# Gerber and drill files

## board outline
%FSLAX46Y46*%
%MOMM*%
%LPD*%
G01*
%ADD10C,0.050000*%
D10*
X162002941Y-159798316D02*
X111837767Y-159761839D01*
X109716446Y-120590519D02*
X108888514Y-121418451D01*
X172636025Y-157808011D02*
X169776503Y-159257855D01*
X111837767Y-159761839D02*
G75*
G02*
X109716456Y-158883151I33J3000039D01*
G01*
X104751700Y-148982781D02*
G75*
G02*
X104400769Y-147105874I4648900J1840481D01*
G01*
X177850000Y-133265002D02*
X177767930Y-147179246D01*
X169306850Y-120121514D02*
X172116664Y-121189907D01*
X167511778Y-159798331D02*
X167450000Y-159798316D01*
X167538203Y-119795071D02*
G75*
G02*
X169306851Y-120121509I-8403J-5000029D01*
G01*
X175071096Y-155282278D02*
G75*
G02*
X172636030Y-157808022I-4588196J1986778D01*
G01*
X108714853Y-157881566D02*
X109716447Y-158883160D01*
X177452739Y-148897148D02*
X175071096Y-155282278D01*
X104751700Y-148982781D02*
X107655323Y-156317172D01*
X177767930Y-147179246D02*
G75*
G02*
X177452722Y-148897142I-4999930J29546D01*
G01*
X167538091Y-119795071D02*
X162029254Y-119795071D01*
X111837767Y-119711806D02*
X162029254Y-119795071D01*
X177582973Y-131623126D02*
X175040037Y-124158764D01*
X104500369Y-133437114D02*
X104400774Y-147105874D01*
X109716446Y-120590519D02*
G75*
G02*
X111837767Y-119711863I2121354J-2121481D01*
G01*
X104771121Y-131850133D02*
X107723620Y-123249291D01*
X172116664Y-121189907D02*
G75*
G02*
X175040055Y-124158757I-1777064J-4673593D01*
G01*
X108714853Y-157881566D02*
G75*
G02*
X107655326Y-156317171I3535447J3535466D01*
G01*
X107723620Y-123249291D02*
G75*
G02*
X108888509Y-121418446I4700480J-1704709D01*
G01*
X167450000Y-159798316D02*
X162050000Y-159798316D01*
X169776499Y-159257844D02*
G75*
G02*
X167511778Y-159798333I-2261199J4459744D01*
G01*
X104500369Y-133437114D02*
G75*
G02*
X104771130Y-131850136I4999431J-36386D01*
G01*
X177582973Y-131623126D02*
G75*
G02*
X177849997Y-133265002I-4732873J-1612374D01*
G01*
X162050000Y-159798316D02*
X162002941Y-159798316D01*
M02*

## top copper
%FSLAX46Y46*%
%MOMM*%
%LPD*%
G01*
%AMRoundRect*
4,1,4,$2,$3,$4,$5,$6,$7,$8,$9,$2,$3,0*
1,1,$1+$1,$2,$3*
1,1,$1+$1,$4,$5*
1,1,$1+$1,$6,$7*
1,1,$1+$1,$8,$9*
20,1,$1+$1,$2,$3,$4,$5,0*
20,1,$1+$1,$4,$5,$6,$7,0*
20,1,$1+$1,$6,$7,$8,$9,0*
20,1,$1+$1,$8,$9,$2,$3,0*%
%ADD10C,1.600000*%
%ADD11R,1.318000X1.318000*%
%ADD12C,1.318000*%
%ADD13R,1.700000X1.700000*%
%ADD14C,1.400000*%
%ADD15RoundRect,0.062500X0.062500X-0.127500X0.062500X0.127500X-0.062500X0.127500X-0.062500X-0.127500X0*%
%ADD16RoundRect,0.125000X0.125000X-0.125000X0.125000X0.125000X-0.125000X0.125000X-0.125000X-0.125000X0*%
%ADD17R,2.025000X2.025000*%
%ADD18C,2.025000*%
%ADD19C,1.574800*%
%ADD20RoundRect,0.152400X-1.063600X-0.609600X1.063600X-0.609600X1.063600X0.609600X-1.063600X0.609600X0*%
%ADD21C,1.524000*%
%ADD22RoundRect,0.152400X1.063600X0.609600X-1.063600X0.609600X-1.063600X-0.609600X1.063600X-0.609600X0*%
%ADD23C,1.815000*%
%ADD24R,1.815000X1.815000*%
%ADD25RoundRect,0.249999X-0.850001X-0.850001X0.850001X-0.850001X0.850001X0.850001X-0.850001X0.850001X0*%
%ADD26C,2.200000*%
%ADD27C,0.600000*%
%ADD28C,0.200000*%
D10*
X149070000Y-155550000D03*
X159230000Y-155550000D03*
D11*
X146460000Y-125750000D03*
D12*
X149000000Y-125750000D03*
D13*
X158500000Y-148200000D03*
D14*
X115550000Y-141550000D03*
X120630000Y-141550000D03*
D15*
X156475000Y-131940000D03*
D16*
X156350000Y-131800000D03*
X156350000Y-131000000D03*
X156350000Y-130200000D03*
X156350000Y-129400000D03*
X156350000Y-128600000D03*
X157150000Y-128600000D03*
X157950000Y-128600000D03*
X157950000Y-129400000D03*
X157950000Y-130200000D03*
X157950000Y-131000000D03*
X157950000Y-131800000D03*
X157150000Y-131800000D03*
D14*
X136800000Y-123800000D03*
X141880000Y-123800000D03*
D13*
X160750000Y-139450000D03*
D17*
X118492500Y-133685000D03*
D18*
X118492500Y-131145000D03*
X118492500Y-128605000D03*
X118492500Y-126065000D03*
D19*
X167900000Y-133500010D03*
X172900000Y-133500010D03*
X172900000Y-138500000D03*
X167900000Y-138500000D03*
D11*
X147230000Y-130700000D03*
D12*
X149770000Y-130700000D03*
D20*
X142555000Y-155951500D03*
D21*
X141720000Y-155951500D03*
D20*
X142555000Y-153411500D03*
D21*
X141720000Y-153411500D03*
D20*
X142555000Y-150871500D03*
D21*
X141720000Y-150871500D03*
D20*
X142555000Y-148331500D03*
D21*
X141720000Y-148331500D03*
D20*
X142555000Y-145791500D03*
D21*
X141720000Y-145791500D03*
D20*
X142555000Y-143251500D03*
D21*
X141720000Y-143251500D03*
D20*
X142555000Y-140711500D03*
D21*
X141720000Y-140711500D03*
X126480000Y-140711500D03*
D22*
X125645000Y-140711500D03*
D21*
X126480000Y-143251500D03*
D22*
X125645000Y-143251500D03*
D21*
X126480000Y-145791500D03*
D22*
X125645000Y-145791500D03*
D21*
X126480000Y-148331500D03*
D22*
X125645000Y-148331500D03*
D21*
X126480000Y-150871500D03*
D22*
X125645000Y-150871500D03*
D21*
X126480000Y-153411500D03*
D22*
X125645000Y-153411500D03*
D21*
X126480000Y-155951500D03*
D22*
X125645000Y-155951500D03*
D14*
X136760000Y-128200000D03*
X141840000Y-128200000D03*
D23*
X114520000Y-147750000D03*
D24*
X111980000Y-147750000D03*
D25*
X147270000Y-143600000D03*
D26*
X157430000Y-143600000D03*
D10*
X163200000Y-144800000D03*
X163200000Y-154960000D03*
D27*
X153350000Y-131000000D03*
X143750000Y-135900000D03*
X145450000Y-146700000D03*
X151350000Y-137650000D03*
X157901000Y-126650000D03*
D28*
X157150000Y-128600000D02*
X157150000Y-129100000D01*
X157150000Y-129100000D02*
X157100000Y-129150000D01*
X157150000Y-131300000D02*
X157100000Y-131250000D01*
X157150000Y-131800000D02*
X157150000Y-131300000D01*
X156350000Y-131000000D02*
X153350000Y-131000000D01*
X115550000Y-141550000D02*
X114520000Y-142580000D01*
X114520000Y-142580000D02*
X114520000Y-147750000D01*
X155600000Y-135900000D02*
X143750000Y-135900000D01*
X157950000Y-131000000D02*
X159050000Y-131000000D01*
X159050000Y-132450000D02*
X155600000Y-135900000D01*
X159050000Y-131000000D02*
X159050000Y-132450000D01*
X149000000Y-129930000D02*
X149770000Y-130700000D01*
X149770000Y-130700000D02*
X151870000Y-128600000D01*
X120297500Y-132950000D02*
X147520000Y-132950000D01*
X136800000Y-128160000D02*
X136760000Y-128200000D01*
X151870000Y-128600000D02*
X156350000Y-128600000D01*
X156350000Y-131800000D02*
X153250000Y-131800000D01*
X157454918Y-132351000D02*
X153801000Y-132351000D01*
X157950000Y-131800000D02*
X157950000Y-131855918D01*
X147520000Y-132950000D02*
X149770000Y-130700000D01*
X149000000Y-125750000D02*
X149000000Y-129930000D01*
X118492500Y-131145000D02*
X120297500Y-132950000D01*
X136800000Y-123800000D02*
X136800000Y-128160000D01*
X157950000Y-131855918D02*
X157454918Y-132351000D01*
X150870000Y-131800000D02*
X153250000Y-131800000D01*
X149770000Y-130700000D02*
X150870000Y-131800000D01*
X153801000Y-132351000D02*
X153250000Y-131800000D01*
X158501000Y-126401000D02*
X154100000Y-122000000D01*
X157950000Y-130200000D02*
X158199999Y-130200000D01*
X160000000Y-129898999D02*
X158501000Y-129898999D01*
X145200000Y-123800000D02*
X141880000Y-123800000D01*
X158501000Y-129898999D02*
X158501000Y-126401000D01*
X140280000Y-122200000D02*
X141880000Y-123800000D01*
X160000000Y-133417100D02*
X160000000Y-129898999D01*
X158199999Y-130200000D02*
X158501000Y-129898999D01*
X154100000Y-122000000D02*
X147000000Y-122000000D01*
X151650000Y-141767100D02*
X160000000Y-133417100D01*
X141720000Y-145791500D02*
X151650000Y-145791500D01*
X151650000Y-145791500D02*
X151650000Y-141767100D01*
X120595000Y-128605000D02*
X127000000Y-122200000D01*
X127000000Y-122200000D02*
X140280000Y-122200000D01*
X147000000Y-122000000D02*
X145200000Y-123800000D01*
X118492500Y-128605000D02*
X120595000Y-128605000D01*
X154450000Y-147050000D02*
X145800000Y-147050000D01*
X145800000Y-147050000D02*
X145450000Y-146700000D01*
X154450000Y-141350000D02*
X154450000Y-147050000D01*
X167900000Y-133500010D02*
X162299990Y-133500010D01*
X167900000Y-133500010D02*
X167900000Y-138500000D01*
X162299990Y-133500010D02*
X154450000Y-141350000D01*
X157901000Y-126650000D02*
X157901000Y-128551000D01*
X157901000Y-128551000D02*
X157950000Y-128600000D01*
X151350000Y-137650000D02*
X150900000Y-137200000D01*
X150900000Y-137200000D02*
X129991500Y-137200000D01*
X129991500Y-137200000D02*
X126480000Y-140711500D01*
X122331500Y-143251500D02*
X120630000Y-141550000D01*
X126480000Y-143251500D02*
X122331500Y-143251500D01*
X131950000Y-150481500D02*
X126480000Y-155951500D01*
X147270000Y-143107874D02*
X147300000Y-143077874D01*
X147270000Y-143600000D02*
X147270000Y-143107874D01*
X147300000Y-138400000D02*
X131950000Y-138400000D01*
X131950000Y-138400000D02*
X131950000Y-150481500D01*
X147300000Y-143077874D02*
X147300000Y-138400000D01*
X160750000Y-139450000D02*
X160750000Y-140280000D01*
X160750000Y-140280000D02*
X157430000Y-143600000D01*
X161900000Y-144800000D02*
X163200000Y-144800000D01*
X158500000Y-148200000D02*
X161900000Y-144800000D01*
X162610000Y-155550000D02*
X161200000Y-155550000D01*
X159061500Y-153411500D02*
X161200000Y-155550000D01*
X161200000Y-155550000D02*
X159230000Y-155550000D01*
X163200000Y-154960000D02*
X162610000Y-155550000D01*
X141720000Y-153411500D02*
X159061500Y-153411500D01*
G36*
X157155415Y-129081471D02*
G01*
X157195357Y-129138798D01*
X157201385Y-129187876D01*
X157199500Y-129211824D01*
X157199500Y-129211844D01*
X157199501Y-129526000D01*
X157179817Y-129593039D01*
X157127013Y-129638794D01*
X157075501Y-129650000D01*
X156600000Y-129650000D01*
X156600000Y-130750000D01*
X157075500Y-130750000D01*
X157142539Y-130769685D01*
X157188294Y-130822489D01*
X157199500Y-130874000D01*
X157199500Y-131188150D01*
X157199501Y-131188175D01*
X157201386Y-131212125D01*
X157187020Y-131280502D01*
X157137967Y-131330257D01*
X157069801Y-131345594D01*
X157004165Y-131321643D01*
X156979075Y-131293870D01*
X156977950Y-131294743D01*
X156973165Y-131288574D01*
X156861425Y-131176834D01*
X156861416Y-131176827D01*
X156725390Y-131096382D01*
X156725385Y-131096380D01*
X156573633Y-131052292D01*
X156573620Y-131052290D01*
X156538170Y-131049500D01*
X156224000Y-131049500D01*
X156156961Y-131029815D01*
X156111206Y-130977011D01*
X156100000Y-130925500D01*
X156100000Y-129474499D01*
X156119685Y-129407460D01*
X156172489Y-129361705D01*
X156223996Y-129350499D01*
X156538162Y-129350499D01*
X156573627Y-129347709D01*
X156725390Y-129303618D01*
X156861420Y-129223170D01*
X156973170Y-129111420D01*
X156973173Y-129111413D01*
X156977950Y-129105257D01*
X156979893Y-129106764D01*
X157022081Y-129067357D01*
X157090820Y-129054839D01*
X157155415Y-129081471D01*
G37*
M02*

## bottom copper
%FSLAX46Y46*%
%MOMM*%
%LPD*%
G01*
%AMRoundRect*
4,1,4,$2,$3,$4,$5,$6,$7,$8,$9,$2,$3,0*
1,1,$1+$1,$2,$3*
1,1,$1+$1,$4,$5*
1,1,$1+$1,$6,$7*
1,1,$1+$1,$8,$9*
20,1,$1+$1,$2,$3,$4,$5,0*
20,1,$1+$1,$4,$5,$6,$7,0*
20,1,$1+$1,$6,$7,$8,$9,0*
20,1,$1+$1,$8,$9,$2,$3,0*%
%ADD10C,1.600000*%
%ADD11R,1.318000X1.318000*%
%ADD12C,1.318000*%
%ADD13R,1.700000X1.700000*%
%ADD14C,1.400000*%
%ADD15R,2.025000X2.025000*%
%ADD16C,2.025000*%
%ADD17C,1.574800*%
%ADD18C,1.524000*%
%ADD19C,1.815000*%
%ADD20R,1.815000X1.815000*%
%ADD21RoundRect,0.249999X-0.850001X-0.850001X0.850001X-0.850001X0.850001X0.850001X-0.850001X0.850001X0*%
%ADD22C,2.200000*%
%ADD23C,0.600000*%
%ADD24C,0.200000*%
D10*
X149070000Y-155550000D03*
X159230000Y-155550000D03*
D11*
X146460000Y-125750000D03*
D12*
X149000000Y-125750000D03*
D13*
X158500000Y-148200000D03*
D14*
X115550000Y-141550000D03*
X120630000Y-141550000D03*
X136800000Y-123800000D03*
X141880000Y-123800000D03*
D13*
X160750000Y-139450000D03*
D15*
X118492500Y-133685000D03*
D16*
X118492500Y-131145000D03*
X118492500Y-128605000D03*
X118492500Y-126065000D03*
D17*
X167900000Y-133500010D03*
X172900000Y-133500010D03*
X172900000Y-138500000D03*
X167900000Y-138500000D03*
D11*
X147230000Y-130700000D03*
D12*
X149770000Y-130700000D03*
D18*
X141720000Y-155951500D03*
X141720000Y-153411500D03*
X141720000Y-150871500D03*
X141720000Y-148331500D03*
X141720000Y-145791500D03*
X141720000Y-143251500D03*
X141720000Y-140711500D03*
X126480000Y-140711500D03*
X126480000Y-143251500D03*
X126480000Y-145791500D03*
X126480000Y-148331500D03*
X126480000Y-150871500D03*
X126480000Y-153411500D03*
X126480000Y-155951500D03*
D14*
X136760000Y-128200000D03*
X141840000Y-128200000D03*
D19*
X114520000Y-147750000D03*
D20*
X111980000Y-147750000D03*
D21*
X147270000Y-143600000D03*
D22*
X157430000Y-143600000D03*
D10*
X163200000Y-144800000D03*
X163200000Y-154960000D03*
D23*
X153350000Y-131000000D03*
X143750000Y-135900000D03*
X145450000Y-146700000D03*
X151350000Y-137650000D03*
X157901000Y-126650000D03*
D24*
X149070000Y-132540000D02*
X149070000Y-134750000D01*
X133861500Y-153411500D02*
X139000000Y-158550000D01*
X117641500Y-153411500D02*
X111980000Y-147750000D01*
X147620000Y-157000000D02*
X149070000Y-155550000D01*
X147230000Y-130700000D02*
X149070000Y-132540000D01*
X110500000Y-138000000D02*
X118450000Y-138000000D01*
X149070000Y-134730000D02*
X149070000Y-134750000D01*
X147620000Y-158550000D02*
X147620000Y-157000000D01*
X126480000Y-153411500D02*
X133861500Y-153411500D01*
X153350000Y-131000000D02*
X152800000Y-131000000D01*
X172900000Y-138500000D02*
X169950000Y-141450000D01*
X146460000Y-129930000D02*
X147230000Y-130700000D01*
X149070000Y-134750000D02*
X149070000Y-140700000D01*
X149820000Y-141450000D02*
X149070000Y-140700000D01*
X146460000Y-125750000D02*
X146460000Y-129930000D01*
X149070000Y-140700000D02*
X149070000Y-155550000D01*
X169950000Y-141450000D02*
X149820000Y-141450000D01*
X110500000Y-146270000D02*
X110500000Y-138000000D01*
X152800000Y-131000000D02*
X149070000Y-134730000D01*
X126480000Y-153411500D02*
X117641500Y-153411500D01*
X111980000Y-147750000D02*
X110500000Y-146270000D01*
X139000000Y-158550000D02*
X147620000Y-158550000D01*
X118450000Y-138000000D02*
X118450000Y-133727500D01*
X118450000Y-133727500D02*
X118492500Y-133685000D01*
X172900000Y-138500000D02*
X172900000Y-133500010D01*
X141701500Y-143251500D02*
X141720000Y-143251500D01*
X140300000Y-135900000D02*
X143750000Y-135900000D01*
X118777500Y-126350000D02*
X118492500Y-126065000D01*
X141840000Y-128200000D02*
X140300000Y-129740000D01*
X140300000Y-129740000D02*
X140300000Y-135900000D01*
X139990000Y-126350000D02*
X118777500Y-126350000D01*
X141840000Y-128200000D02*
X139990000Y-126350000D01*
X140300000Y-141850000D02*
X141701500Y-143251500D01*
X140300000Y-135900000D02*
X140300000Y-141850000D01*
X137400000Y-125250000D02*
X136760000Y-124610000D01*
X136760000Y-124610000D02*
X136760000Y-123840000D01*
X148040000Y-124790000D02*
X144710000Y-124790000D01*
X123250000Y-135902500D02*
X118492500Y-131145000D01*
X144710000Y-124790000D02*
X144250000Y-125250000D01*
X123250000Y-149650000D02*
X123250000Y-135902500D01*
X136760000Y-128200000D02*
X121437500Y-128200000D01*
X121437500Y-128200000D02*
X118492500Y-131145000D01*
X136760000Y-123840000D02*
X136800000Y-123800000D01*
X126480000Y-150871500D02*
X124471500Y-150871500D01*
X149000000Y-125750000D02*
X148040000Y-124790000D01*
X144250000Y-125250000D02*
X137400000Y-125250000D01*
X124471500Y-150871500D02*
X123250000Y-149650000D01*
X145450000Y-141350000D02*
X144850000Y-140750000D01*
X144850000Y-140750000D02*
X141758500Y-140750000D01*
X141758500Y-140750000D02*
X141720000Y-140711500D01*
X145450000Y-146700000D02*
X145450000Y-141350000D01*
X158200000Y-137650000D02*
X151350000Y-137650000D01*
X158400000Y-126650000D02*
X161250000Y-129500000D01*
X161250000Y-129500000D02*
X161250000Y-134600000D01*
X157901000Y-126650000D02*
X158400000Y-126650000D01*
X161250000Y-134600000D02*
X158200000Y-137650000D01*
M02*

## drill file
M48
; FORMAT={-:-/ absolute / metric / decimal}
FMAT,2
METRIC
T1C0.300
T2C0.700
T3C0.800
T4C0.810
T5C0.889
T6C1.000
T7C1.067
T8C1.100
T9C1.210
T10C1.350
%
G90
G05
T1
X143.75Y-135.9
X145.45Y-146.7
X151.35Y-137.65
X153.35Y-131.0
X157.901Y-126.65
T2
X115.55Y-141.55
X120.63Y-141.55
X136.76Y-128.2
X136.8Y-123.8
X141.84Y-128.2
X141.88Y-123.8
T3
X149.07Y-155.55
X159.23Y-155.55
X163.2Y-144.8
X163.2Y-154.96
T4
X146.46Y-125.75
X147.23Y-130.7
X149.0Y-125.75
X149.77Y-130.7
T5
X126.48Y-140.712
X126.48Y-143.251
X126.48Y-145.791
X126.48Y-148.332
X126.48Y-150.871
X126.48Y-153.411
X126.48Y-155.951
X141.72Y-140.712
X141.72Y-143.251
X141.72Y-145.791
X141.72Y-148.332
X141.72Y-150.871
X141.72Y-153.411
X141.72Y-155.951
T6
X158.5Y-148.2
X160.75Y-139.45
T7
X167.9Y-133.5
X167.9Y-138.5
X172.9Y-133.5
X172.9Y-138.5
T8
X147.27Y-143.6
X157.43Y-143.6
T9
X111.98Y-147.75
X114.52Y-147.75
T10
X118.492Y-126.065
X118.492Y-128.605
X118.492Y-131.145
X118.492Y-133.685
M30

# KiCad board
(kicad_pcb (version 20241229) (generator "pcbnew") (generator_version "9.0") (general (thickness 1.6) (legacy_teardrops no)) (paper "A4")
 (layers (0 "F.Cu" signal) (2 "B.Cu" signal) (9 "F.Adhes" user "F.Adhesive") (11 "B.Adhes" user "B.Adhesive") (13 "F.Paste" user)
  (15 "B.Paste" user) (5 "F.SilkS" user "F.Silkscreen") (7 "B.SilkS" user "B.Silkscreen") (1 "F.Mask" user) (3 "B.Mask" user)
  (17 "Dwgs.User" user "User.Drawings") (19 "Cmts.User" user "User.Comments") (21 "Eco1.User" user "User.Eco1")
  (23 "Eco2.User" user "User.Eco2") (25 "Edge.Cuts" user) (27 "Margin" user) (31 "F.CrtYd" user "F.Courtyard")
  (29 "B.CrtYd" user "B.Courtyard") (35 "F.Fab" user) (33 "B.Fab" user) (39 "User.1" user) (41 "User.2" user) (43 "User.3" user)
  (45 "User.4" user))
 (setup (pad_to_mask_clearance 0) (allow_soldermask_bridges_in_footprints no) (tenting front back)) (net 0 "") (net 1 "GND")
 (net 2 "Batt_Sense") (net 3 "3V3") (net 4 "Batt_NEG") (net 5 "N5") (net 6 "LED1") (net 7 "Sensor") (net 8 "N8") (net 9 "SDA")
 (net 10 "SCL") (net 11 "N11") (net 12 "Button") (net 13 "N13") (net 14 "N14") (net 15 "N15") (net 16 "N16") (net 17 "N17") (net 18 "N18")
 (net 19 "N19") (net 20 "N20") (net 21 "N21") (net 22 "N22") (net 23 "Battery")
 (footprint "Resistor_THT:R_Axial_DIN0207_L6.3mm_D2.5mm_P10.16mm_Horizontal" (layer "F.Cu") (at 149.07 155.55)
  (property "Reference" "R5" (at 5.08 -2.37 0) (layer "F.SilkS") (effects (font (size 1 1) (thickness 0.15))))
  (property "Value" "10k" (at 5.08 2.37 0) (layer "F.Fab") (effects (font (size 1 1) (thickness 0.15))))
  (pad "1" thru_hole circle (at 0 0) (size 1.6 1.6) (drill 0.8) (layers "*.Cu" "*.Mask") (remove_unused_layers no) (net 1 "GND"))
  (pad "2" thru_hole circle (at 10.16 0) (size 1.6 1.6) (drill 0.8) (layers "*.Cu" "*.Mask") (remove_unused_layers no) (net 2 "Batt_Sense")))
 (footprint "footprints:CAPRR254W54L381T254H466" (layer "F.Cu") (at 147.73 125.75)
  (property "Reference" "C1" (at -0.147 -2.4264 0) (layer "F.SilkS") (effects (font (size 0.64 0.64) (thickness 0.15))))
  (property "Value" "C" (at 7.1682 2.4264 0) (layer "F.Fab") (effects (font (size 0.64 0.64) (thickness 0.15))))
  (pad "1" thru_hole rect (at -1.27 0) (size 1.318 1.318) (drill 0.81) (layers "*.Cu" "*.Mask") (remove_unused_layers no) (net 1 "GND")
   (solder_mask_margin 0.102))
  (pad "2" thru_hole circle (at 1.27 0) (size 1.318 1.318) (drill 0.81) (layers "*.Cu" "*.Mask") (remove_unused_layers no) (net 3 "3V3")
   (solder_mask_margin 0.102)))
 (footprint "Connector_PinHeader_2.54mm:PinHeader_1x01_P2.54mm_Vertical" (layer "F.Cu") (at 158.5 148.2)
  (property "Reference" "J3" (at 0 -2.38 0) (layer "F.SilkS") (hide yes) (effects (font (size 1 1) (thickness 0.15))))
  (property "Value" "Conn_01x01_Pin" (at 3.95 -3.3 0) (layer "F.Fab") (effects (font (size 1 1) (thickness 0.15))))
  (pad "1" thru_hole rect (at 0 0) (size 1.7 1.7) (drill 1) (layers "*.Cu" "*.Mask") (remove_unused_layers no) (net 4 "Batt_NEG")))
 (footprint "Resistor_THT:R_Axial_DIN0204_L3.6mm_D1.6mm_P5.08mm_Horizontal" (layer "F.Cu") (at 115.55 141.55)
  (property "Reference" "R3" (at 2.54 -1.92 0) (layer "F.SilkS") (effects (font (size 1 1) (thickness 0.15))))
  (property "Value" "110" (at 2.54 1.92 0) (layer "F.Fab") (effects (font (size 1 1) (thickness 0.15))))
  (pad "1" thru_hole circle (at 0 0) (size 1.4 1.4) (drill 0.7) (layers "*.Cu" "*.Mask") (remove_unused_layers no) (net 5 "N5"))
  (pad "2" thru_hole circle (at 5.08 0) (size 1.4 1.4) (drill 0.7) (layers "*.Cu" "*.Mask") (remove_unused_layers no) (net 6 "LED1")))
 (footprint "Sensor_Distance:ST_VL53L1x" (layer "F.Cu") (at 157.15 130.2 90)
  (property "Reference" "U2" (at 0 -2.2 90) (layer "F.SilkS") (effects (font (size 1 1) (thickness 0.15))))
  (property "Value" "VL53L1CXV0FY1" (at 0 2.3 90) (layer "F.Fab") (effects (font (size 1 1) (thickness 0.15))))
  (pad "1" smd roundrect (at -1.74 -0.675 90) (size 0.38 0.25) (layers "F.Cu" "F.Mask" "F.Paste") (roundrect_rratio 0.25) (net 3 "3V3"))
  (pad "1" smd roundrect (at -1.6 -0.8 90) (size 0.5 0.5) (layers "F.Cu" "F.Mask" "F.Paste") (roundrect_rratio 0.25) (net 3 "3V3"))
  (pad "2" smd roundrect (at -0.8 -0.8 90) (size 0.5 0.5) (layers "F.Cu" "F.Mask" "F.Paste") (roundrect_rratio 0.25) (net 1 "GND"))
  (pad "3" smd roundrect (at 0 -0.8 90) (size 0.5 0.5) (layers "F.Cu" "F.Mask" "F.Paste") (roundrect_rratio 0.25) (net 1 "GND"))
  (pad "4" smd roundrect (at 0.8 -0.8 90) (size 0.5 0.5) (layers "F.Cu" "F.Mask" "F.Paste") (roundrect_rratio 0.25) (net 1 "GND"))
  (pad "5" smd roundrect (at 1.6 -0.8 90) (size 0.5 0.5) (layers "F.Cu" "F.Mask" "F.Paste") (roundrect_rratio 0.25) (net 3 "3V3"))
  (pad "6" smd roundrect (at 1.6 0 90) (size 0.5 0.5) (layers "F.Cu" "F.Mask" "F.Paste") (roundrect_rratio 0.25) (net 1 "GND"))
  (pad "7" smd roundrect (at 1.6 0.8 90) (size 0.5 0.5) (layers "F.Cu" "F.Mask" "F.Paste") (roundrect_rratio 0.25) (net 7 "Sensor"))
  (pad "8" smd roundrect (at 0.8 0.8 90) (size 0.5 0.5) (layers "F.Cu" "F.Mask" "F.Paste") (roundrect_rratio 0.25) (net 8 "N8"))
  (pad "9" smd roundrect (at 0 0.8 90) (size 0.5 0.5) (layers "F.Cu" "F.Mask" "F.Paste") (roundrect_rratio 0.25) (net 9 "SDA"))
  (pad "10" smd roundrect (at -0.8 0.8 90) (size 0.5 0.5) (layers "F.Cu" "F.Mask" "F.Paste") (roundrect_rratio 0.25) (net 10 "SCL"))
  (pad "11" smd roundrect (at -1.6 0.8 90) (size 0.5 0.5) (layers "F.Cu" "F.Mask" "F.Paste") (roundrect_rratio 0.25) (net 3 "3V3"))
  (pad "12" smd roundrect (at -1.6 0 90) (size 0.5 0.5) (layers "F.Cu" "F.Mask" "F.Paste") (roundrect_rratio 0.25) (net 1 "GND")))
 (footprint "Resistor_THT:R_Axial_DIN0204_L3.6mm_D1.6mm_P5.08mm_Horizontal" (layer "F.Cu") (at 136.8 123.8)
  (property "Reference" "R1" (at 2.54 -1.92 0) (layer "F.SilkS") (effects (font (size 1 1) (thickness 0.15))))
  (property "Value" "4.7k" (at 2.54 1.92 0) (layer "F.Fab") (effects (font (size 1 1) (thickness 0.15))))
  (pad "1" thru_hole circle (at 0 0) (size 1.4 1.4) (drill 0.7) (layers "*.Cu" "*.Mask") (remove_unused_layers no) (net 3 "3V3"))
  (pad "2" thru_hole circle (at 5.08 0) (size 1.4 1.4) (drill 0.7) (layers "*.Cu" "*.Mask") (remove_unused_layers no) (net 9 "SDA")))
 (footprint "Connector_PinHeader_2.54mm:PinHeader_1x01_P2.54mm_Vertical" (layer "F.Cu") (at 160.75 139.45)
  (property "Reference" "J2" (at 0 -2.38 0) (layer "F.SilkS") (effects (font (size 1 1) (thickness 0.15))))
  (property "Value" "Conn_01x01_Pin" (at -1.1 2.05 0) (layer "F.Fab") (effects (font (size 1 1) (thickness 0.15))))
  (pad "1" thru_hole rect (at 0 0) (size 1.7 1.7) (drill 1) (layers "*.Cu" "*.Mask") (remove_unused_layers no) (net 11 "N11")))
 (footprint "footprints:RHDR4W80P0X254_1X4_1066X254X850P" (layer "F.Cu") (at 118.4925 133.685 90)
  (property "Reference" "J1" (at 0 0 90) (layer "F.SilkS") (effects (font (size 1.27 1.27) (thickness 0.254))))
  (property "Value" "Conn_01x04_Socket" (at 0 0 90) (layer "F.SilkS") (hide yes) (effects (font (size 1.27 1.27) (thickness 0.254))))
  (pad "1" thru_hole rect (at 0 0 90) (size 2.025 2.025) (drill 1.35) (layers "*.Cu" "*.Mask") (remove_unused_layers no) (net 1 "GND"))
  (pad "2" thru_hole circle (at 2.54 0 90) (size 2.025 2.025) (drill 1.35) (layers "*.Cu" "*.Mask") (remove_unused_layers no) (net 3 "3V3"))
  (pad "3" thru_hole circle (at 5.08 0 90) (size 2.025 2.025) (drill 1.35) (layers "*.Cu" "*.Mask") (remove_unused_layers no) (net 9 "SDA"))
  (pad "4" thru_hole circle (at 7.62 0 90) (size 2.025 2.025) (drill 1.35) (layers "*.Cu" "*.Mask") (remove_unused_layers no) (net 10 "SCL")))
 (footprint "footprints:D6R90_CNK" (layer "F.Cu") (at 167.9 133.50001)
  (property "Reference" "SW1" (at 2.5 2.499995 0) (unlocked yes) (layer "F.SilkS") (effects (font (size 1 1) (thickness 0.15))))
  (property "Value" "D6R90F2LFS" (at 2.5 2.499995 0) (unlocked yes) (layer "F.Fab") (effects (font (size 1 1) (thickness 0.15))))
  (pad "1" thru_hole circle (at 0 0) (size 1.5748 1.5748) (drill 1.0668) (layers "*.Cu" "*.Mask") (remove_unused_layers no)
   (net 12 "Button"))
  (pad "2" thru_hole circle (at 5 0) (size 1.5748 1.5748) (drill 1.0668) (layers "*.Cu" "*.Mask") (remove_unused_layers no) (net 1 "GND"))
  (pad "3" thru_hole circle (at 5 4.99999) (size 1.5748 1.5748) (drill 1.0668) (layers "*.Cu" "*.Mask") (remove_unused_layers no)
   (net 1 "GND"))
  (pad "4" thru_hole circle (at 0 4.99999) (size 1.5748 1.5748) (drill 1.0668) (layers "*.Cu" "*.Mask") (remove_unused_layers no)
   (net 12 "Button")))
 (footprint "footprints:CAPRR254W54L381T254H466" (layer "F.Cu") (at 148.5 130.7)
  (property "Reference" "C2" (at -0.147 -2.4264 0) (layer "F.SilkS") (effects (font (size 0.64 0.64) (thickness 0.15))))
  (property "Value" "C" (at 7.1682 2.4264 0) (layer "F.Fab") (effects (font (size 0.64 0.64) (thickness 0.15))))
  (pad "1" thru_hole rect (at -1.27 0) (size 1.318 1.318) (drill 0.81) (layers "*.Cu" "*.Mask") (remove_unused_layers no) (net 1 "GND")
   (solder_mask_margin 0.102))
  (pad "2" thru_hole circle (at 1.27 0) (size 1.318 1.318) (drill 0.81) (layers "*.Cu" "*.Mask") (remove_unused_layers no) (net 3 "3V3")
   (solder_mask_margin 0.102)))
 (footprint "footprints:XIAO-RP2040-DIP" (layer "F.Cu") (at 134.1 148.3315 -90)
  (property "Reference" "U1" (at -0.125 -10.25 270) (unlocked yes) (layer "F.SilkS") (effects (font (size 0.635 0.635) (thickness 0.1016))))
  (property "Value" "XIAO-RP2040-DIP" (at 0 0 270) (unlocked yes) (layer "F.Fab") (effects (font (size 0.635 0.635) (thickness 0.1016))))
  (pad "1" smd roundrect (at 7.62 -8.455) (size 2.432 1.524) (layers "F.Cu" "F.Mask") (roundrect_rratio 0.1) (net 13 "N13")
   (thermal_bridge_angle 45))
  (pad "1" thru_hole circle (at 7.62 -7.62) (size 1.524 1.524) (drill 0.889) (layers "*.Cu" "*.Mask") (remove_unused_layers no)
   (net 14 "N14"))
  (pad "2" smd roundrect (at 5.08 -8.455) (size 2.432 1.524) (layers "F.Cu" "F.Mask") (roundrect_rratio 0.1) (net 2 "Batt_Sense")
   (thermal_bridge_angle 45))
  (pad "2" thru_hole circle (at 5.08 -7.62) (size 1.524 1.524) (drill 0.889) (layers "*.Cu" "*.Mask") (remove_unused_layers no)
   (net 2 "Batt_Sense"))
  (pad "3" smd roundrect (at 2.54 -8.455) (size 2.432 1.524) (layers "F.Cu" "F.Mask") (roundrect_rratio 0.1) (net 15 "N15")
   (thermal_bridge_angle 45))
  (pad "3" thru_hole circle (at 2.54 -7.62) (size 1.524 1.524) (drill 0.889) (layers "*.Cu" "*.Mask") (remove_unused_layers no)
   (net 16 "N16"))
  (pad "4" smd roundrect (at 0 -8.455) (size 2.432 1.524) (layers "F.Cu" "F.Mask") (roundrect_rratio 0.1) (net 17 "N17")
   (thermal_bridge_angle 45))
  (pad "4" thru_hole circle (at 0 -7.62) (size 1.524 1.524) (drill 0.889) (layers "*.Cu" "*.Mask") (remove_unused_layers no) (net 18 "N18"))
  (pad "5" smd roundrect (at -2.54 -8.455) (size 2.432 1.524) (layers "F.Cu" "F.Mask") (roundrect_rratio 0.1) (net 9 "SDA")
   (thermal_bridge_angle 45))
  (pad "5" thru_hole circle (at -2.54 -7.62) (size 1.524 1.524) (drill 0.889) (layers "*.Cu" "*.Mask") (remove_unused_layers no)
   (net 9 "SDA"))
  (pad "6" smd roundrect (at -5.08 -8.455) (size 2.432 1.524) (layers "F.Cu" "F.Mask") (roundrect_rratio 0.1) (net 10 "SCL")
   (thermal_bridge_angle 45))
  (pad "6" thru_hole circle (at -5.08 -7.62) (size 1.524 1.524) (drill 0.889) (layers "*.Cu" "*.Mask") (remove_unused_layers no)
   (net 10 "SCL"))
  (pad "7" smd roundrect (at -7.62 -8.455) (size 2.432 1.524) (layers "F.Cu" "F.Mask") (roundrect_rratio 0.1) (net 12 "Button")
   (thermal_bridge_angle 45))
  (pad "7" thru_hole circle (at -7.62 -7.62) (size 1.524 1.524) (drill 0.889) (layers "*.Cu" "*.Mask") (remove_unused_layers no)
   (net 12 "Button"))
  (pad "8" thru_hole circle (at -7.62 7.62 180) (size 1.524 1.524) (drill 0.889) (layers "*.Cu" "*.Mask") (remove_unused_layers no)
   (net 7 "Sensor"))
  (pad "8" smd roundrect (at -7.62 8.455 180) (size 2.432 1.524) (layers "F.Cu" "F.Mask") (roundrect_rratio 0.1) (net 7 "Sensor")
   (thermal_bridge_angle 45))
  (pad "9" thru_hole circle (at -5.08 7.62 180) (size 1.524 1.524) (drill 0.889) (layers "*.Cu" "*.Mask") (remove_unused_layers no)
   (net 6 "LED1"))
  (pad "9" smd roundrect (at -5.08 8.455 180) (size 2.432 1.524) (layers "F.Cu" "F.Mask") (roundrect_rratio 0.1) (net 6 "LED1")
   (thermal_bridge_angle 45))
  (pad "10" thru_hole circle (at -2.54 7.62 180) (size 1.524 1.524) (drill 0.889) (layers "*.Cu" "*.Mask") (remove_unused_layers no)
   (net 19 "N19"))
  (pad "10" smd roundrect (at -2.54 8.455 180) (size 2.432 1.524) (layers "F.Cu" "F.Mask") (roundrect_rratio 0.1) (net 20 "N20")
   (thermal_bridge_angle 45))
  (pad "11" thru_hole circle (at 0 7.62 180) (size 1.524 1.524) (drill 0.889) (layers "*.Cu" "*.Mask") (remove_unused_layers no)
   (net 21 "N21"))
  (pad "11" smd roundrect (at 0 8.455 180) (size 2.432 1.524) (layers "F.Cu" "F.Mask") (roundrect_rratio 0.1) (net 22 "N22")
   (thermal_bridge_angle 45))
  (pad "12" thru_hole circle (at 2.54 7.62 180) (size 1.524 1.524) (drill 0.889) (layers "*.Cu" "*.Mask") (remove_unused_layers no)
   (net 3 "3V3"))
  (pad "12" smd roundrect (at 2.54 8.455 180) (size 2.432 1.524) (layers "F.Cu" "F.Mask") (roundrect_rratio 0.1) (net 3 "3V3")
   (thermal_bridge_angle 45))
  (pad "13" thru_hole circle (at 5.08 7.62 180) (size 1.524 1.524) (drill 0.889) (layers "*.Cu" "*.Mask") (remove_unused_layers no)
   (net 1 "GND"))
  (pad "13" smd roundrect (at 5.08 8.455 180) (size 2.432 1.524) (layers "F.Cu" "F.Mask") (roundrect_rratio 0.1) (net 1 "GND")
   (thermal_bridge_angle 45))
  (pad "14" thru_hole circle (at 7.62 7.62 180) (size 1.524 1.524) (drill 0.889) (layers "*.Cu" "*.Mask") (remove_unused_layers no)
   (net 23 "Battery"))
  (pad "14" smd roundrect (at 7.62 8.455 180) (size 2.432 1.524) (layers "F.Cu" "F.Mask") (roundrect_rratio 0.1) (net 23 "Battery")
   (thermal_bridge_angle 45)))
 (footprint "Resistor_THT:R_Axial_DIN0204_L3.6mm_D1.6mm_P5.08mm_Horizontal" (layer "F.Cu") (at 136.76 128.2)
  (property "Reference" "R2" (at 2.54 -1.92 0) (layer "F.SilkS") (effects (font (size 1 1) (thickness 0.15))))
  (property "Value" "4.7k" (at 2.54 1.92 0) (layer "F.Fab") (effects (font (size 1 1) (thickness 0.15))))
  (pad "1" thru_hole circle (at 0 0) (size 1.4 1.4) (drill 0.7) (layers "*.Cu" "*.Mask") (remove_unused_layers no) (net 3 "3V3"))
  (pad "2" thru_hole circle (at 5.08 0) (size 1.4 1.4) (drill 0.7) (layers "*.Cu" "*.Mask") (remove_unused_layers no) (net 10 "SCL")))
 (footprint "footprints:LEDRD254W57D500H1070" (layer "F.Cu") (at 113.25 147.75)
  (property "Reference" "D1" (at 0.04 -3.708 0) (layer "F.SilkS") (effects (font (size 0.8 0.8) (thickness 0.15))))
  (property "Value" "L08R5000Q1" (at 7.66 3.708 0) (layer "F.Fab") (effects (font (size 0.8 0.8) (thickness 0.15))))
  (pad "A" thru_hole circle (at 1.27 0) (size 1.815 1.815) (drill 1.21) (layers "*.Cu" "*.Mask") (remove_unused_layers no) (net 5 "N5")
   (solder_mask_margin 0.102))
  (pad "C" thru_hole rect (at -1.27 0) (size 1.815 1.815) (drill 1.21) (layers "*.Cu" "*.Mask") (remove_unused_layers no) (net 1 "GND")
   (solder_mask_margin 0.102)))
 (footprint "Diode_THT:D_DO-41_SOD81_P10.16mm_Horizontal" (layer "F.Cu") (at 147.27 143.6)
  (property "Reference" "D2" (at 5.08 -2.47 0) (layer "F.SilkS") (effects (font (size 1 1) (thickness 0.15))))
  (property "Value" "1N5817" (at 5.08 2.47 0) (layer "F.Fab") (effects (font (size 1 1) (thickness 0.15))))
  (pad "1" thru_hole roundrect (at 0 0) (size 2.2 2.2) (drill 1.1) (layers "*.Cu" "*.Mask") (remove_unused_layers no)
   (roundrect_rratio 0.113636) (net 23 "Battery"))
  (pad "2" thru_hole circle (at 10.16 0) (size 2.2 2.2) (drill 1.1) (layers "*.Cu" "*.Mask") (remove_unused_layers no) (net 11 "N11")))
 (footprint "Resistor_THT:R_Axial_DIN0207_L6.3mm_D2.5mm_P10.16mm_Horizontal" (layer "F.Cu") (at 163.2 144.8 -90)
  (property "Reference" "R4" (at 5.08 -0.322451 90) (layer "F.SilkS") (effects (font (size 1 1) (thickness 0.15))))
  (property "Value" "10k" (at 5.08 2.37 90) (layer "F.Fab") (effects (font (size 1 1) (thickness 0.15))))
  (pad "1" thru_hole circle (at 0 0 270) (size 1.6 1.6) (drill 0.8) (layers "*.Cu" "*.Mask") (remove_unused_layers no) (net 4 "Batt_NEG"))
  (pad "2" thru_hole circle (at 10.16 0 270) (size 1.6 1.6) (drill 0.8) (layers "*.Cu" "*.Mask") (remove_unused_layers no)
   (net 2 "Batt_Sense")))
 (gr_line (start 162.002941 159.798316) (end 111.837767 159.761839) (stroke (width 0.05) (type default)) (layer "Edge.Cuts"))
 (gr_line (start 109.716446 120.590519) (end 108.888514 121.418451) (stroke (width 0.05) (type default)) (layer "Edge.Cuts"))
 (gr_line (start 172.636025 157.808011) (end 169.776503 159.257855) (stroke (width 0.05) (type default)) (layer "Edge.Cuts"))
 (gr_arc (start 111.837767 159.761839) (mid 110.689717 159.533478) (end 109.716447 158.88316) (stroke (width 0.05) (type default))
  (layer "Edge.Cuts"))
 (gr_arc (start 104.7517 148.982781) (mid 104.485809 148.061235) (end 104.400774 147.105874) (stroke (width 0.05) (type default))
  (layer "Edge.Cuts"))
 (gr_line (start 177.85 133.265002) (end 177.76793 147.179246) (stroke (width 0.05) (type default)) (layer "Edge.Cuts"))
 (gr_line (start 169.30685 120.121514) (end 172.116664 121.189907) (stroke (width 0.05) (type default)) (layer "Edge.Cuts"))
 (gr_line (start 167.511778 159.798331) (end 167.45 159.798316) (stroke (width 0.05) (type default)) (layer "Edge.Cuts"))
 (gr_arc (start 167.538203 119.795071) (mid 168.437327 119.878107) (end 169.306856 120.121497) (stroke (width 0.05) (type default))
  (layer "Edge.Cuts"))
 (gr_arc (start 175.071096 155.282278) (mid 174.08237 156.765741) (end 172.636025 157.808011) (stroke (width 0.05) (type default))
  (layer "Edge.Cuts"))
 (gr_line (start 108.714853 157.881566) (end 109.716447 158.88316) (stroke (width 0.05) (type default)) (layer "Edge.Cuts"))
 (gr_line (start 177.452739 148.897148) (end 175.071096 155.282278) (stroke (width 0.05) (type default)) (layer "Edge.Cuts"))
 (gr_line (start 104.7517 148.982781) (end 107.655323 156.317172) (stroke (width 0.05) (type default)) (layer "Edge.Cuts"))
 (gr_arc (start 177.76793 147.179246) (mid 177.685926 148.052065) (end 177.452739 148.897148) (stroke (width 0.05) (type default))
  (layer "Edge.Cuts"))
 (gr_line (start 167.538091 119.795071) (end 162.029254 119.795071) (stroke (width 0.05) (type default)) (layer "Edge.Cuts"))
 (gr_line (start 111.837767 119.711806) (end 162.029254 119.795071) (stroke (width 0.05) (type default)) (layer "Edge.Cuts"))
 (gr_line (start 177.582973 131.623126) (end 175.040037 124.158764) (stroke (width 0.05) (type default)) (layer "Edge.Cuts"))
 (gr_line (start 104.500369 133.437114) (end 104.400774 147.105874) (stroke (width 0.05) (type default)) (layer "Edge.Cuts"))
 (gr_arc (start 109.716446 120.590519) (mid 110.689719 119.940214) (end 111.837767 119.711839) (stroke (width 0.05) (type default))
  (layer "Edge.Cuts"))
 (gr_line (start 104.771121 131.850133) (end 107.72362 123.249291) (stroke (width 0.05) (type default)) (layer "Edge.Cuts"))
 (gr_arc (start 172.116664 121.189907) (mid 173.902325 122.355321) (end 175.040037 124.158764) (stroke (width 0.05) (type default))
  (layer "Edge.Cuts"))
 (gr_arc (start 108.714853 157.881566) (mid 108.110519 157.149873) (end 107.655323 156.317172) (stroke (width 0.05) (type default))
  (layer "Edge.Cuts"))
 (gr_arc (start 107.72362 123.249291) (mid 108.205546 122.269913) (end 108.888514 121.418451) (stroke (width 0.05) (type default))
  (layer "Edge.Cuts"))
 (gr_line (start 167.45 159.798316) (end 162.05 159.798316) (stroke (width 0.05) (type default)) (layer "Edge.Cuts"))
 (gr_arc (start 169.776499 159.257844) (mid 168.676035 159.661735) (end 167.511778 159.798316) (stroke (width 0.05) (type default))
  (layer "Edge.Cuts"))
 (gr_arc (start 104.500369 133.437114) (mid 104.571447 132.632653) (end 104.771121 131.850133) (stroke (width 0.05) (type default))
  (layer "Edge.Cuts"))
 (gr_arc (start 177.582973 131.623126) (mid 177.785245 132.432881) (end 177.85 133.265002) (stroke (width 0.05) (type default))
  (layer "Edge.Cuts"))
 (gr_line (start 162.05 159.798316) (end 162.002941 159.798316) (stroke (width 0.05) (type default)) (layer "Edge.Cuts"))
 (segment (start 157.15 128.6) (end 157.15 129.1) (width 0.2) (layer "F.Cu") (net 1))
 (segment (start 157.15 129.1) (end 157.1 129.15) (width 0.2) (layer "F.Cu") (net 1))
 (segment (start 157.15 131.3) (end 157.1 131.25) (width 0.2) (layer "F.Cu") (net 1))
 (segment (start 157.15 131.8) (end 157.15 131.3) (width 0.2) (layer "F.Cu") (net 1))
 (segment (start 156.35 131) (end 153.35 131) (width 0.2) (layer "F.Cu") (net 1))
 (via (at 153.35 131) (size 0.6) (drill 0.3) (layers "F.Cu" "B.Cu") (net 1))
 (segment (start 149.07 132.54) (end 149.07 134.75) (width 0.2) (layer "B.Cu") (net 1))
 (segment (start 133.8615 153.4115) (end 139 158.55) (width 0.2) (layer "B.Cu") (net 1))
 (segment (start 117.6415 153.4115) (end 111.98 147.75) (width 0.2) (layer "B.Cu") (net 1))
 (segment (start 147.62 157) (end 149.07 155.55) (width 0.2) (layer "B.Cu") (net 1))
 (segment (start 147.23 130.7) (end 149.07 132.54) (width 0.2) (layer "B.Cu") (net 1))
 (segment (start 110.5 138) (end 118.45 138) (width 0.2) (layer "B.Cu") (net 1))
 (segment (start 149.07 134.73) (end 149.07 134.75) (width 0.2) (layer "B.Cu") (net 1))
 (segment (start 147.62 158.55) (end 147.62 157) (width 0.2) (layer "B.Cu") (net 1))
 (segment (start 126.48 153.4115) (end 133.8615 153.4115) (width 0.2) (layer "B.Cu") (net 1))
 (segment (start 153.35 131) (end 152.8 131) (width 0.2) (layer "B.Cu") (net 1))
 (segment (start 172.9 138.5) (end 169.95 141.45) (width 0.2) (layer "B.Cu") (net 1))
 (segment (start 146.46 129.93) (end 147.23 130.7) (width 0.2) (layer "B.Cu") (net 1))
 (segment (start 149.07 134.75) (end 149.07 140.7) (width 0.2) (layer "B.Cu") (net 1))
 (segment (start 149.82 141.45) (end 149.07 140.7) (width 0.2) (layer "B.Cu") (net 1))
 (segment (start 146.46 125.75) (end 146.46 129.93) (width 0.2) (layer "B.Cu") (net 1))
 (segment (start 149.07 140.7) (end 149.07 155.55) (width 0.2) (layer "B.Cu") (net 1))
 (segment (start 169.95 141.45) (end 149.82 141.45) (width 0.2) (layer "B.Cu") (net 1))
 (segment (start 110.5 146.27) (end 110.5 138) (width 0.2) (layer "B.Cu") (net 1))
 (segment (start 152.8 131) (end 149.07 134.73) (width 0.2) (layer "B.Cu") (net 1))
 (segment (start 126.48 153.4115) (end 117.6415 153.4115) (width 0.2) (layer "B.Cu") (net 1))
 (segment (start 111.98 147.75) (end 110.5 146.27) (width 0.2) (layer "B.Cu") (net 1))
 (segment (start 139 158.55) (end 147.62 158.55) (width 0.2) (layer "B.Cu") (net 1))
 (segment (start 118.45 138) (end 118.45 133.7275) (width 0.2) (layer "B.Cu") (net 1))
 (segment (start 118.45 133.7275) (end 118.4925 133.685) (width 0.2) (layer "B.Cu") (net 1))
 (segment (start 172.9 138.5) (end 172.9 133.50001) (width 0.2) (layer "B.Cu") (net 1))
 (segment (start 115.55 141.55) (end 114.52 142.58) (width 0.2) (layer "F.Cu") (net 5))
 (segment (start 114.52 142.58) (end 114.52 147.75) (width 0.2) (layer "F.Cu") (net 5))
 (segment (start 155.6 135.9) (end 143.75 135.9) (width 0.2) (layer "F.Cu") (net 10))
 (segment (start 157.95 131) (end 159.05 131) (width 0.2) (layer "F.Cu") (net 10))
 (segment (start 159.05 132.45) (end 155.6 135.9) (width 0.2) (layer "F.Cu") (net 10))
 (segment (start 159.05 131) (end 159.05 132.45) (width 0.2) (layer "F.Cu") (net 10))
 (via (at 143.75 135.9) (size 0.6) (drill 0.3) (layers "F.Cu" "B.Cu") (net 10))
 (segment (start 141.7015 143.2515) (end 141.72 143.2515) (width 0.2) (layer "B.Cu") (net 10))
 (segment (start 140.3 135.9) (end 143.75 135.9) (width 0.2) (layer "B.Cu") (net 10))
 (segment (start 118.7775 126.35) (end 118.4925 126.065) (width 0.2) (layer "B.Cu") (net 10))
 (segment (start 141.84 128.2) (end 140.3 129.74) (width 0.2) (layer "B.Cu") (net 10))
 (segment (start 140.3 129.74) (end 140.3 135.9) (width 0.2) (layer "B.Cu") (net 10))
 (segment (start 139.99 126.35) (end 118.7775 126.35) (width 0.2) (layer "B.Cu") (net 10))
 (segment (start 141.84 128.2) (end 139.99 126.35) (width 0.2) (layer "B.Cu") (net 10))
 (segment (start 140.3 141.85) (end 141.7015 143.2515) (width 0.2) (layer "B.Cu") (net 10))
 (segment (start 140.3 135.9) (end 140.3 141.85) (width 0.2) (layer "B.Cu") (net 10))
 (segment (start 149 129.93) (end 149.77 130.7) (width 0.2) (layer "F.Cu") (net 3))
 (segment (start 149.77 130.7) (end 151.87 128.6) (width 0.2) (layer "F.Cu") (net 3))
 (segment (start 120.2975 132.95) (end 147.52 132.95) (width 0.2) (layer "F.Cu") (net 3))
 (segment (start 136.8 128.16) (end 136.76 128.2) (width 0.2) (layer "F.Cu") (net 3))
 (segment (start 151.87 128.6) (end 156.35 128.6) (width 0.2) (layer "F.Cu") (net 3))
 (segment (start 156.35 131.8) (end 153.25 131.8) (width 0.2) (layer "F.Cu") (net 3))
 (segment (start 157.454918 132.351) (end 153.801 132.351) (width 0.2) (layer "F.Cu") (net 3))
 (segment (start 157.95 131.8) (end 157.95 131.855918) (width 0.2) (layer "F.Cu") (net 3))
 (segment (start 147.52 132.95) (end 149.77 130.7) (width 0.2) (layer "F.Cu") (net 3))
 (segment (start 149 125.75) (end 149 129.93) (width 0.2) (layer "F.Cu") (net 3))
 (segment (start 118.4925 131.145) (end 120.2975 132.95) (width 0.2) (layer "F.Cu") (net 3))
 (segment (start 136.8 123.8) (end 136.8 128.16) (width 0.2) (layer "F.Cu") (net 3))
 (segment (start 157.95 131.855918) (end 157.454918 132.351) (width 0.2) (layer "F.Cu") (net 3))
 (segment (start 150.87 131.8) (end 153.25 131.8) (width 0.2) (layer "F.Cu") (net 3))
 (segment (start 149.77 130.7) (end 150.87 131.8) (width 0.2) (layer "F.Cu") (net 3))
 (segment (start 153.801 132.351) (end 153.25 131.8) (width 0.2) (layer "F.Cu") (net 3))
 (segment (start 137.4 125.25) (end 136.76 124.61) (width 0.2) (layer "B.Cu") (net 3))
 (segment (start 136.76 124.61) (end 136.76 123.84) (width 0.2) (layer "B.Cu") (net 3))
 (segment (start 148.04 124.79) (end 144.71 124.79) (width 0.2) (layer "B.Cu") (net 3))
 (segment (start 123.25 135.9025) (end 118.4925 131.145) (width 0.2) (layer "B.Cu") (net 3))
 (segment (start 144.71 124.79) (end 144.25 125.25) (width 0.2) (layer "B.Cu") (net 3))
 (segment (start 123.25 149.65) (end 123.25 135.9025) (width 0.2) (layer "B.Cu") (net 3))
 (segment (start 136.76 128.2) (end 121.4375 128.2) (width 0.2) (layer "B.Cu") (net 3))
 (segment (start 121.4375 128.2) (end 118.4925 131.145) (width 0.2) (layer "B.Cu") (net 3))
 (segment (start 136.76 123.84) (end 136.8 123.8) (width 0.2) (layer "B.Cu") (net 3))
 (segment (start 126.48 150.8715) (end 124.4715 150.8715) (width 0.2) (layer "B.Cu") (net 3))
 (segment (start 149 125.75) (end 148.04 124.79) (width 0.2) (layer "B.Cu") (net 3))
 (segment (start 144.25 125.25) (end 137.4 125.25) (width 0.2) (layer "B.Cu") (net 3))
 (segment (start 124.4715 150.8715) (end 123.25 149.65) (width 0.2) (layer "B.Cu") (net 3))
 (segment (start 158.501 126.401) (end 154.1 122) (width 0.2) (layer "F.Cu") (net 9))
 (segment (start 157.95 130.2) (end 158.199999 130.2) (width 0.2) (layer "F.Cu") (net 9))
 (segment (start 160 129.898999) (end 158.501 129.898999) (width 0.2) (layer "F.Cu") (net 9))
 (segment (start 145.2 123.8) (end 141.88 123.8) (width 0.2) (layer "F.Cu") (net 9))
 (segment (start 158.501 129.898999) (end 158.501 126.401) (width 0.2) (layer "F.Cu") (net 9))
 (segment (start 140.28 122.2) (end 141.88 123.8) (width 0.2) (layer "F.Cu") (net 9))
 (segment (start 160 133.4171) (end 160 129.898999) (width 0.2) (layer "F.Cu") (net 9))
 (segment (start 158.199999 130.2) (end 158.501 129.898999) (width 0.2) (layer "F.Cu") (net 9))
 (segment (start 154.1 122) (end 147 122) (width 0.2) (layer "F.Cu") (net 9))
 (segment (start 151.65 141.7671) (end 160 133.4171) (width 0.2) (layer "F.Cu") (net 9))
 (segment (start 141.72 145.7915) (end 151.65 145.7915) (width 0.2) (layer "F.Cu") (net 9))
 (segment (start 151.65 145.7915) (end 151.65 141.7671) (width 0.2) (layer "F.Cu") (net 9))
 (segment (start 120.595 128.605) (end 127 122.2) (width 0.2) (layer "F.Cu") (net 9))
 (segment (start 127 122.2) (end 140.28 122.2) (width 0.2) (layer "F.Cu") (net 9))
 (segment (start 147 122) (end 145.2 123.8) (width 0.2) (layer "F.Cu") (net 9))
 (segment (start 118.4925 128.605) (end 120.595 128.605) (width 0.2) (layer "F.Cu") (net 9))
 (segment (start 154.45 147.05) (end 145.8 147.05) (width 0.2) (layer "F.Cu") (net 12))
 (segment (start 145.8 147.05) (end 145.45 146.7) (width 0.2) (layer "F.Cu") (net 12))
 (segment (start 154.45 141.35) (end 154.45 147.05) (width 0.2) (layer "F.Cu") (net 12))
 (segment (start 167.9 133.50001) (end 162.29999 133.50001) (width 0.2) (layer "F.Cu") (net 12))
 (segment (start 167.9 133.50001) (end 167.9 138.5) (width 0.2) (layer "F.Cu") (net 12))
 (segment (start 162.29999 133.50001) (end 154.45 141.35) (width 0.2) (layer "F.Cu") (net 12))
 (via (at 145.45 146.7) (size 0.6) (drill 0.3) (layers "F.Cu" "B.Cu") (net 12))
 (segment (start 145.45 141.35) (end 144.85 140.75) (width 0.2) (layer "B.Cu") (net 12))
 (segment (start 144.85 140.75) (end 141.7585 140.75) (width 0.2) (layer "B.Cu") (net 12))
 (segment (start 141.7585 140.75) (end 141.72 140.7115) (width 0.2) (layer "B.Cu") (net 12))
 (segment (start 145.45 146.7) (end 145.45 141.35) (width 0.2) (layer "B.Cu") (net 12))
 (segment (start 157.901 126.65) (end 157.901 128.551) (width 0.2) (layer "F.Cu") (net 7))
 (segment (start 157.901 128.551) (end 157.95 128.6) (width 0.2) (layer "F.Cu") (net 7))
 (segment (start 151.35 137.65) (end 150.9 137.2) (width 0.2) (layer "F.Cu") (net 7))
 (segment (start 150.9 137.2) (end 129.9915 137.2) (width 0.2) (layer "F.Cu") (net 7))
 (segment (start 129.9915 137.2) (end 126.48 140.7115) (width 0.2) (layer "F.Cu") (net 7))
 (via (at 151.35 137.65) (size 0.6) (drill 0.3) (layers "F.Cu" "B.Cu") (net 7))
 (via (at 157.901 126.65) (size 0.6) (drill 0.3) (layers "F.Cu" "B.Cu") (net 7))
 (segment (start 158.2 137.65) (end 151.35 137.65) (width 0.2) (layer "B.Cu") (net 7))
 (segment (start 158.4 126.65) (end 161.25 129.5) (width 0.2) (layer "B.Cu") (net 7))
 (segment (start 161.25 129.5) (end 161.25 134.6) (width 0.2) (layer "B.Cu") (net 7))
 (segment (start 157.901 126.65) (end 158.4 126.65) (width 0.2) (layer "B.Cu") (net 7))
 (segment (start 161.25 134.6) (end 158.2 137.65) (width 0.2) (layer "B.Cu") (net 7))
 (segment (start 122.3315 143.2515) (end 120.63 141.55) (width 0.2) (layer "F.Cu") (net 6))
 (segment (start 126.48 143.2515) (end 122.3315 143.2515) (width 0.2) (layer "F.Cu") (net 6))
 (segment (start 131.95 150.4815) (end 126.48 155.9515) (width 0.2) (layer "F.Cu") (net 23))
 (segment (start 147.27 143.107874) (end 147.3 143.077874) (width 0.2) (layer "F.Cu") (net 23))
 (segment (start 147.27 143.6) (end 147.27 143.107874) (width 0.2) (layer "F.Cu") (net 23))
 (segment (start 147.3 138.4) (end 131.95 138.4) (width 0.2) (layer "F.Cu") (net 23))
 (segment (start 131.95 138.4) (end 131.95 150.4815) (width 0.2) (layer "F.Cu") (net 23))
 (segment (start 147.3 143.077874) (end 147.3 138.4) (width 0.2) (layer "F.Cu") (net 23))
 (segment (start 160.75 139.45) (end 160.75 140.28) (width 0.2) (layer "F.Cu") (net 11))
 (segment (start 160.75 140.28) (end 157.43 143.6) (width 0.2) (layer "F.Cu") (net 11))
 (segment (start 161.9 144.8) (end 163.2 144.8) (width 0.2) (layer "F.Cu") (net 4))
 (segment (start 158.5 148.2) (end 161.9 144.8) (width 0.2) (layer "F.Cu") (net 4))
 (segment (start 162.61 155.55) (end 161.2 155.55) (width 0.2) (layer "F.Cu") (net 2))
 (segment (start 159.0615 153.4115) (end 161.2 155.55) (width 0.2) (layer "F.Cu") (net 2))
 (segment (start 161.2 155.55) (end 159.23 155.55) (width 0.2) (layer "F.Cu") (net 2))
 (segment (start 163.2 154.96) (end 162.61 155.55) (width 0.2) (layer "F.Cu") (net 2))
 (segment (start 141.72 153.4115) (end 159.0615 153.4115) (width 0.2) (layer "F.Cu") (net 2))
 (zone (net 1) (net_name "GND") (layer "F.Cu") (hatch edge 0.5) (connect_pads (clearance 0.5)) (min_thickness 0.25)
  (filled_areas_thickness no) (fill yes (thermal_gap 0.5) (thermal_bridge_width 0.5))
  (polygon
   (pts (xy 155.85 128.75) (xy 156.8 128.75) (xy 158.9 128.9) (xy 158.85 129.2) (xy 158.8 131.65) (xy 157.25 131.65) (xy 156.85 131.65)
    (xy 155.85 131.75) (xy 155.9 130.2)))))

